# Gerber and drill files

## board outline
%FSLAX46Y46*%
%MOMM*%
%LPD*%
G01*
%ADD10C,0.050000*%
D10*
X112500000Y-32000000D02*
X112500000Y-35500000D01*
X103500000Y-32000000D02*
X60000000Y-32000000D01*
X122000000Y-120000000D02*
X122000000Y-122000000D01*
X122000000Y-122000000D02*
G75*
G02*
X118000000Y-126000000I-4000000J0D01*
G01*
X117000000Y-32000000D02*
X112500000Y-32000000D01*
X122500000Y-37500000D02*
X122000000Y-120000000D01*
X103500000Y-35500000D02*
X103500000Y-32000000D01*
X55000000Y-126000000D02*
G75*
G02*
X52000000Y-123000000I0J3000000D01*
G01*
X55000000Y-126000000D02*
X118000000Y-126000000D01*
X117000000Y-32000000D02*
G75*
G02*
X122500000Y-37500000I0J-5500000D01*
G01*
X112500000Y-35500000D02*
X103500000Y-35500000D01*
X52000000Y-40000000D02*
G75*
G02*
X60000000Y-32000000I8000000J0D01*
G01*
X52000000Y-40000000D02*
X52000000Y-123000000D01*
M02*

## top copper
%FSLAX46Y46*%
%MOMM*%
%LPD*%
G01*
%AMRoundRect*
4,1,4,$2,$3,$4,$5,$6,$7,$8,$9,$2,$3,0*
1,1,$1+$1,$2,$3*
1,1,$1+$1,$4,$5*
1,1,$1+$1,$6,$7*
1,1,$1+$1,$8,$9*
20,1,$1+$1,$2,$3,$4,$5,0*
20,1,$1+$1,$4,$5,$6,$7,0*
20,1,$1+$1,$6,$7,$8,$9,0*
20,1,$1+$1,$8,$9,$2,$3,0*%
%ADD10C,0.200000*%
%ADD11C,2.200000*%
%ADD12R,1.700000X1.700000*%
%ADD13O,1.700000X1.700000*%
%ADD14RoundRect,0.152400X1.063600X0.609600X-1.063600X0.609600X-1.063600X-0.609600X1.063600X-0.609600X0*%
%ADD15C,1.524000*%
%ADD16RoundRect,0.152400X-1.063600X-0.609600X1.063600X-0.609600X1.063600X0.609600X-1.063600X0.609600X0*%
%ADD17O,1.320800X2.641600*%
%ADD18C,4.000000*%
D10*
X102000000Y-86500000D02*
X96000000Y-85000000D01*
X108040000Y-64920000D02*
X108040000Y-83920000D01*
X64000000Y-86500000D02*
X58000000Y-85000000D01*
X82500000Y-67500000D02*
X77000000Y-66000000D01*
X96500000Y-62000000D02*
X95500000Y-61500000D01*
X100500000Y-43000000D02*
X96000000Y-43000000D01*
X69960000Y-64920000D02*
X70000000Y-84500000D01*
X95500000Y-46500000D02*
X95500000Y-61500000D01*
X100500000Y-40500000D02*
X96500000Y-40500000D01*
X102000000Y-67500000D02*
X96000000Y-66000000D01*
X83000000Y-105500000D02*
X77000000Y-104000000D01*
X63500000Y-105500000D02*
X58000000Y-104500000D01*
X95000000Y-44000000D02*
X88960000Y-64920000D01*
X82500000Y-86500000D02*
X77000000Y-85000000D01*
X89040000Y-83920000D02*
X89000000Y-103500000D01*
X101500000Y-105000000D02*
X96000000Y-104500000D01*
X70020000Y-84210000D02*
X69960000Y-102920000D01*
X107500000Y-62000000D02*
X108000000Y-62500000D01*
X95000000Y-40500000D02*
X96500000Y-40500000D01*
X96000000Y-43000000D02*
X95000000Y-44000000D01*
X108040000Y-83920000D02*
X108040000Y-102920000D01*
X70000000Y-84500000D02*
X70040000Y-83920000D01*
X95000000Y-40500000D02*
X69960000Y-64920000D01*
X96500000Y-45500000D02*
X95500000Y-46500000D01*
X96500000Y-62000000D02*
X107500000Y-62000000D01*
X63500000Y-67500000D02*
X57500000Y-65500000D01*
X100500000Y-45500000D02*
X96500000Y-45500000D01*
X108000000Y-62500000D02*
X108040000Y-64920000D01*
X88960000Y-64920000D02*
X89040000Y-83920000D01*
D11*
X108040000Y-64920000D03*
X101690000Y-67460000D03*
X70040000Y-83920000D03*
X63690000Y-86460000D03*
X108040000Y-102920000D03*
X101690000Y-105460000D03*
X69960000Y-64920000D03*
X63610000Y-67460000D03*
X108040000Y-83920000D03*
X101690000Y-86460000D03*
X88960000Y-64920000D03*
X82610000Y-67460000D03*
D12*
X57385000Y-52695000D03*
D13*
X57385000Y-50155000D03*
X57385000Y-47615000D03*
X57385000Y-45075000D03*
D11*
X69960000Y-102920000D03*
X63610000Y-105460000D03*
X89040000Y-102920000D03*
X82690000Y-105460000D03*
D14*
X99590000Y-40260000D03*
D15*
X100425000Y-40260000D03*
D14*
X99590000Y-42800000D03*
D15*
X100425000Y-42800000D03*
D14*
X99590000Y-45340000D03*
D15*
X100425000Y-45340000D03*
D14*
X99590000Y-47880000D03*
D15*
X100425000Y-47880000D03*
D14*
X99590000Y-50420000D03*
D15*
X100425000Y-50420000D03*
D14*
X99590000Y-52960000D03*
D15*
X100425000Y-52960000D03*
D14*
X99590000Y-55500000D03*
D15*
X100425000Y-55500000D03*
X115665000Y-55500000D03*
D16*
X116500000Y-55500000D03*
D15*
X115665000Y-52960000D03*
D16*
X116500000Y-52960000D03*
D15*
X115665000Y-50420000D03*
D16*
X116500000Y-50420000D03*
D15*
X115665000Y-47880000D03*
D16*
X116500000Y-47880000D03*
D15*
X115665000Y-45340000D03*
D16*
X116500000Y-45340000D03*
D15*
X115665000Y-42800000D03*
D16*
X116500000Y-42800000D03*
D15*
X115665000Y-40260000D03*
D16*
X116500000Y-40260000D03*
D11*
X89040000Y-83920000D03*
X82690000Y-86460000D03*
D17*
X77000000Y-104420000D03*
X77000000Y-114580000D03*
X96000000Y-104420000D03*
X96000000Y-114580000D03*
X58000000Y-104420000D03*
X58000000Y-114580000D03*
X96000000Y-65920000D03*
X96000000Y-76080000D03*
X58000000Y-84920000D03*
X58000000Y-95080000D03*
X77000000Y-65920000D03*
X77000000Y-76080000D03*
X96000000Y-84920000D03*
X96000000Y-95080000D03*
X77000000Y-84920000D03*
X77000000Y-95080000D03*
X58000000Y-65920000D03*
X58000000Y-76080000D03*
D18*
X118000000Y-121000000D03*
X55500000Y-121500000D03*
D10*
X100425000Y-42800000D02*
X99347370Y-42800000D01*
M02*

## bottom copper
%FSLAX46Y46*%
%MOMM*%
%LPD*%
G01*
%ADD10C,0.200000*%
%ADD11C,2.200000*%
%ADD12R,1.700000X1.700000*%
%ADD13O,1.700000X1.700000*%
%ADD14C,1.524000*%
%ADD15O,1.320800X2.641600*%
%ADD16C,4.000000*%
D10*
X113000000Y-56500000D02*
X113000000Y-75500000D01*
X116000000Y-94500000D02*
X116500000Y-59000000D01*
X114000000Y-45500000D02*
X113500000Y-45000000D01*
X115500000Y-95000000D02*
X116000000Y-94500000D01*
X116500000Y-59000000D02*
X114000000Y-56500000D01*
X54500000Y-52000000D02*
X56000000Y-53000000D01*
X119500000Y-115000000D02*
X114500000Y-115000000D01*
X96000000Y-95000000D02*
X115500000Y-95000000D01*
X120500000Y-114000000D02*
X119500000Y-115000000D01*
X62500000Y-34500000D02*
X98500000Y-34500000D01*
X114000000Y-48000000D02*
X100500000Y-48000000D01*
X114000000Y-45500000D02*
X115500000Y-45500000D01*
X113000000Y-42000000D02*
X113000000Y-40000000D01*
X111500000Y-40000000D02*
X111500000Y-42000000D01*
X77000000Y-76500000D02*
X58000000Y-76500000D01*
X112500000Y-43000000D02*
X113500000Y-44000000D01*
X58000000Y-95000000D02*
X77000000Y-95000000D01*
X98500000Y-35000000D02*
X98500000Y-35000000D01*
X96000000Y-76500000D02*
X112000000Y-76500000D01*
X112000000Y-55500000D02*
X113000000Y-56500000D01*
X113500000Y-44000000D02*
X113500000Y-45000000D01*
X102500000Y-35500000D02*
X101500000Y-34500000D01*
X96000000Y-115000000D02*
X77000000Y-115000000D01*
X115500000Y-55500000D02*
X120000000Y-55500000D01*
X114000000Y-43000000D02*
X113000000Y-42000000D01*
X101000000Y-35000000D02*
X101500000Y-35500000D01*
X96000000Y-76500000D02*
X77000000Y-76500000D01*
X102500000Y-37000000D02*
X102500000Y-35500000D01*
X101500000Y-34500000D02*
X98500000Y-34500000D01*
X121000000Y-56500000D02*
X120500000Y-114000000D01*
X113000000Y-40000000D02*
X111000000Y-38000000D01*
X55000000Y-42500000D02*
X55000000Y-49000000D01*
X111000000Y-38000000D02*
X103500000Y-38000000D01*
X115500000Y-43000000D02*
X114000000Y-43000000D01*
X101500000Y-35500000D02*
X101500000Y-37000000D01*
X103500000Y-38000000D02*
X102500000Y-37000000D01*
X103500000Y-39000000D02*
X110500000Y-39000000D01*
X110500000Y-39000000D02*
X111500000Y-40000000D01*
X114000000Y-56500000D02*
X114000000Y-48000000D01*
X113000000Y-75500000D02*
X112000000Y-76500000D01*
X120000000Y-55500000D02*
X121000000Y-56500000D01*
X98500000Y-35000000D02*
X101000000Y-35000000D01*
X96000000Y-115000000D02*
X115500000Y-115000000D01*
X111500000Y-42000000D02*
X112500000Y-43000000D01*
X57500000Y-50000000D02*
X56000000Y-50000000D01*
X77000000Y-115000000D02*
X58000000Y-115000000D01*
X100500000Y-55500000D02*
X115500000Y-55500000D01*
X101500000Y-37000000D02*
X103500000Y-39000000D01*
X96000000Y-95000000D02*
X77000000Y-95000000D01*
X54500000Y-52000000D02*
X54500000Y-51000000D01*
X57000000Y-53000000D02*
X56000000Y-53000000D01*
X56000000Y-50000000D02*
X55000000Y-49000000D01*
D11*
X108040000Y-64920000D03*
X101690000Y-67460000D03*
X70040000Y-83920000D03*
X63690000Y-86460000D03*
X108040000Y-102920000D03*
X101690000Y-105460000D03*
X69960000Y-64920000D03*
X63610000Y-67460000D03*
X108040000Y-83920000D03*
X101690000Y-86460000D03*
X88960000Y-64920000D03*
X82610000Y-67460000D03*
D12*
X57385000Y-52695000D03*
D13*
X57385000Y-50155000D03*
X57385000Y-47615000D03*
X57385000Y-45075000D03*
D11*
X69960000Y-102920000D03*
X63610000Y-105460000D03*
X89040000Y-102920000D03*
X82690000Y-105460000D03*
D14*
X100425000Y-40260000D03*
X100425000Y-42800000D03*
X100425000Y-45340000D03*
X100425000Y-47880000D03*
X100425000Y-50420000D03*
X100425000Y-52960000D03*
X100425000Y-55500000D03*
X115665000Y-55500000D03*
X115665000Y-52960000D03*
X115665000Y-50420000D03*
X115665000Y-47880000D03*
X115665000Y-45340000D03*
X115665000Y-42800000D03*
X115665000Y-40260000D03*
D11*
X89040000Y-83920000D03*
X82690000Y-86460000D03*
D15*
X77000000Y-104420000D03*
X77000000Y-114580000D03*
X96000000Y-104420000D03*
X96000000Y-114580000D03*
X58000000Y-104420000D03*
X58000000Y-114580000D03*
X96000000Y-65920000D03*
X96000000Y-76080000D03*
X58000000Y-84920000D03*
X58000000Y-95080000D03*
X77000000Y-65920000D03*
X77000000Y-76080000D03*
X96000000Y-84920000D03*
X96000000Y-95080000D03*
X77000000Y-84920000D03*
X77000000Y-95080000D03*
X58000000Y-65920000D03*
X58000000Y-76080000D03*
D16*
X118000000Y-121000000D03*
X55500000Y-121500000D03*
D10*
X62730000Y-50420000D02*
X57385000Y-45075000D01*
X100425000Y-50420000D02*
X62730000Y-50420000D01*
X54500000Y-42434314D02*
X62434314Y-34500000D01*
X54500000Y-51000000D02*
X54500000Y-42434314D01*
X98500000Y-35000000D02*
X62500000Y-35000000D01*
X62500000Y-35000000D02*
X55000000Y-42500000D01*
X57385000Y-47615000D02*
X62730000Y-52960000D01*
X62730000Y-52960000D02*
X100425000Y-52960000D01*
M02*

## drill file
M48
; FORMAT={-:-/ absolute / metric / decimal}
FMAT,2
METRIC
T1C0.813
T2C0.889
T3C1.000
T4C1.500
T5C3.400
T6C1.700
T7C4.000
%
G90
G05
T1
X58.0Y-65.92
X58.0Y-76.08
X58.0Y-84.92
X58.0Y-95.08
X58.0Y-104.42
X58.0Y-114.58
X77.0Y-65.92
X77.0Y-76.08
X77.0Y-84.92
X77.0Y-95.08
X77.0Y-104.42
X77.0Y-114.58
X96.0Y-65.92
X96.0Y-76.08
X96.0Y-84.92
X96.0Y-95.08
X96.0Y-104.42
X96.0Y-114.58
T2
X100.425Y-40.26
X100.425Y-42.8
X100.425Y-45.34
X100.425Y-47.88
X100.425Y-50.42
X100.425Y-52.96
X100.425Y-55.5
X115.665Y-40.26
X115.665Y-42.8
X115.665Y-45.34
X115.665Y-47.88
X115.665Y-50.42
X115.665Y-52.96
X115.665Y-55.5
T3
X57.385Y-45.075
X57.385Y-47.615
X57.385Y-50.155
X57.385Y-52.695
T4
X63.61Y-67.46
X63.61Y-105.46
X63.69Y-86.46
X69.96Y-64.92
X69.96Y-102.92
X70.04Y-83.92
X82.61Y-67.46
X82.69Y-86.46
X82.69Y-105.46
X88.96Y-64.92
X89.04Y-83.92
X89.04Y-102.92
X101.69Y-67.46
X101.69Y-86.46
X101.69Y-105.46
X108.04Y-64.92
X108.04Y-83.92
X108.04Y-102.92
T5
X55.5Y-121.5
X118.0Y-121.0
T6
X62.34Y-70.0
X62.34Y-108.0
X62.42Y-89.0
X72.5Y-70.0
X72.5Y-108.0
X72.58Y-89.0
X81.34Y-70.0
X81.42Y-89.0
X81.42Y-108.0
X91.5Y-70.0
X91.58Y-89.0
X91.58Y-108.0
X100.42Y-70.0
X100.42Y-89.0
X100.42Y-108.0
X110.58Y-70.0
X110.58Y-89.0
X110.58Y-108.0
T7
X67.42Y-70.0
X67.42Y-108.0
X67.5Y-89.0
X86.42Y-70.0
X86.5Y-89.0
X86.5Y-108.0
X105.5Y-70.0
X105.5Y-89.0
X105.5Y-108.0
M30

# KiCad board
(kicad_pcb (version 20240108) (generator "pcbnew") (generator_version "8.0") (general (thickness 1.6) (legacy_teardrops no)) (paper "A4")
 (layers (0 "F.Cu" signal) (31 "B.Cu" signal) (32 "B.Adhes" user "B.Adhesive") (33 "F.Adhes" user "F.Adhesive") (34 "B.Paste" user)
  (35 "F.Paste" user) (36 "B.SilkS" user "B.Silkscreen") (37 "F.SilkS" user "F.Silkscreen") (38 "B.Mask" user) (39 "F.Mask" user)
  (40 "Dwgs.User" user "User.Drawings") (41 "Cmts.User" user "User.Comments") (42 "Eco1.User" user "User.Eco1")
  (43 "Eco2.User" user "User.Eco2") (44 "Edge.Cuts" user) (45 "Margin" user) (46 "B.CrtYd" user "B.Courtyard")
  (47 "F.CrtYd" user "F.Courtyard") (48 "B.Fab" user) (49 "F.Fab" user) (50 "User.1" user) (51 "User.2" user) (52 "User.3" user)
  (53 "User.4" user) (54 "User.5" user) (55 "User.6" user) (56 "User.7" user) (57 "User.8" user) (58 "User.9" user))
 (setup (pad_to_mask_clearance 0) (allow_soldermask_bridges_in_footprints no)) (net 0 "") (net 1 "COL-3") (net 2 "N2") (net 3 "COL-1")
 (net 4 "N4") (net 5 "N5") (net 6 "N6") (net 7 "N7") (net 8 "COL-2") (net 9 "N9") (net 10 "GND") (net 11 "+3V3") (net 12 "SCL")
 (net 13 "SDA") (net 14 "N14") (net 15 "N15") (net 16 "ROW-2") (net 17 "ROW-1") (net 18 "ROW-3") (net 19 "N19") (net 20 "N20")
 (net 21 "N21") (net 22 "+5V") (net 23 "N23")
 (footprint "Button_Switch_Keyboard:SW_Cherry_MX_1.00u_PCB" (layer "F.Cu") (at 108.04 64.92)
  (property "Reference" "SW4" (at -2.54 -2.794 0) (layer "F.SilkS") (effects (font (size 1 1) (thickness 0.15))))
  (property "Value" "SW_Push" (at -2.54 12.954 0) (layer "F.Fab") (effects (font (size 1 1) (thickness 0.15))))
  (pad "" np_thru_hole circle (at -7.62 5.08) (size 1.7 1.7) (drill 1.7) (layers "*.Cu" "*.Mask"))
  (pad "" np_thru_hole circle (at -2.54 5.08) (size 4 4) (drill 4) (layers "*.Cu" "*.Mask"))
  (pad "" np_thru_hole circle (at 2.54 5.08) (size 1.7 1.7) (drill 1.7) (layers "*.Cu" "*.Mask"))
  (pad "1" thru_hole circle (at 0 0) (size 2.2 2.2) (drill 1.5) (layers "*.Cu" "*.Mask") (remove_unused_layers no) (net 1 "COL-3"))
  (pad "2" thru_hole circle (at -6.35 2.54) (size 2.2 2.2) (drill 1.5) (layers "*.Cu" "*.Mask") (remove_unused_layers no) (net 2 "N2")))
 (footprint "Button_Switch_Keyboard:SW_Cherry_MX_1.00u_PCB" (layer "F.Cu") (at 70.04 83.92)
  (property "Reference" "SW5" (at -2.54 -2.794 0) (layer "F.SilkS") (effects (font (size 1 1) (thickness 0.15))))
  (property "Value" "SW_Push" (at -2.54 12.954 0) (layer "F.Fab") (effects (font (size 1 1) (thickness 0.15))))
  (pad "" np_thru_hole circle (at -7.62 5.08) (size 1.7 1.7) (drill 1.7) (layers "*.Cu" "*.Mask"))
  (pad "" np_thru_hole circle (at -2.54 5.08) (size 4 4) (drill 4) (layers "*.Cu" "*.Mask"))
  (pad "" np_thru_hole circle (at 2.54 5.08) (size 1.7 1.7) (drill 1.7) (layers "*.Cu" "*.Mask"))
  (pad "1" thru_hole circle (at 0 0) (size 2.2 2.2) (drill 1.5) (layers "*.Cu" "*.Mask") (remove_unused_layers no) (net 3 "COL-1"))
  (pad "2" thru_hole circle (at -6.35 2.54) (size 2.2 2.2) (drill 1.5) (layers "*.Cu" "*.Mask") (remove_unused_layers no) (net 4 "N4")))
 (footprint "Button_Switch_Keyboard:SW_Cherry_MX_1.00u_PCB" (layer "F.Cu") (at 108.04 102.92)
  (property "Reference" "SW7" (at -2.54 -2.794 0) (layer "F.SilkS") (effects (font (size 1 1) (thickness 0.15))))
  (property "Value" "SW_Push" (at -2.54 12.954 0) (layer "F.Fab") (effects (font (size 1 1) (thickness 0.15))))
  (pad "" np_thru_hole circle (at -7.62 5.08) (size 1.7 1.7) (drill 1.7) (layers "*.Cu" "*.Mask"))
  (pad "" np_thru_hole circle (at -2.54 5.08) (size 4 4) (drill 4) (layers "*.Cu" "*.Mask"))
  (pad "" np_thru_hole circle (at 2.54 5.08) (size 1.7 1.7) (drill 1.7) (layers "*.Cu" "*.Mask"))
  (pad "1" thru_hole circle (at 0 0) (size 2.2 2.2) (drill 1.5) (layers "*.Cu" "*.Mask") (remove_unused_layers no) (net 1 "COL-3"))
  (pad "2" thru_hole circle (at -6.35 2.54) (size 2.2 2.2) (drill 1.5) (layers "*.Cu" "*.Mask") (remove_unused_layers no) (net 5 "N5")))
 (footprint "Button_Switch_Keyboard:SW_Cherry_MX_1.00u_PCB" (layer "F.Cu") (at 69.96 64.92)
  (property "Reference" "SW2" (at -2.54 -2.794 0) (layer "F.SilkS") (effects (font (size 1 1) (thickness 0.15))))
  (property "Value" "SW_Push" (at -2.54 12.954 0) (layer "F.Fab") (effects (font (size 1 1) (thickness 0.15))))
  (pad "" np_thru_hole circle (at -7.62 5.08) (size 1.7 1.7) (drill 1.7) (layers "*.Cu" "*.Mask"))
  (pad "" np_thru_hole circle (at -2.54 5.08) (size 4 4) (drill 4) (layers "*.Cu" "*.Mask"))
  (pad "" np_thru_hole circle (at 2.54 5.08) (size 1.7 1.7) (drill 1.7) (layers "*.Cu" "*.Mask"))
  (pad "1" thru_hole circle (at 0 0) (size 2.2 2.2) (drill 1.5) (layers "*.Cu" "*.Mask") (remove_unused_layers no) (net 3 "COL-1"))
  (pad "2" thru_hole circle (at -6.35 2.54) (size 2.2 2.2) (drill 1.5) (layers "*.Cu" "*.Mask") (remove_unused_layers no) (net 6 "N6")))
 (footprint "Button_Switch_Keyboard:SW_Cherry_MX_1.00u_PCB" (layer "F.Cu") (at 108.04 83.92)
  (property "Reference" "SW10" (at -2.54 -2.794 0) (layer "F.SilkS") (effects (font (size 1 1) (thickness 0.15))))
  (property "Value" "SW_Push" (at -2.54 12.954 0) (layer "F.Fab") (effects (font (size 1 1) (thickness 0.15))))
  (pad "" np_thru_hole circle (at -7.62 5.08) (size 1.7 1.7) (drill 1.7) (layers "*.Cu" "*.Mask"))
  (pad "" np_thru_hole circle (at -2.54 5.08) (size 4 4) (drill 4) (layers "*.Cu" "*.Mask"))
  (pad "" np_thru_hole circle (at 2.54 5.08) (size 1.7 1.7) (drill 1.7) (layers "*.Cu" "*.Mask"))
  (pad "1" thru_hole circle (at 0 0) (size 2.2 2.2) (drill 1.5) (layers "*.Cu" "*.Mask") (remove_unused_layers no) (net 1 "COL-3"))
  (pad "2" thru_hole circle (at -6.35 2.54) (size 2.2 2.2) (drill 1.5) (layers "*.Cu" "*.Mask") (remove_unused_layers no) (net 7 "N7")))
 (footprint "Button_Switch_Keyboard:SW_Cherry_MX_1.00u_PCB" (layer "F.Cu") (at 88.96 64.92)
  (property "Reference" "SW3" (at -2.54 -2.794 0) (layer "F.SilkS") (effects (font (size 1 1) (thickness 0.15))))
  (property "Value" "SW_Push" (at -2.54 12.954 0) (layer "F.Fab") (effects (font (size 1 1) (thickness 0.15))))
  (pad "" np_thru_hole circle (at -7.62 5.08) (size 1.7 1.7) (drill 1.7) (layers "*.Cu" "*.Mask"))
  (pad "" np_thru_hole circle (at -2.54 5.08) (size 4 4) (drill 4) (layers "*.Cu" "*.Mask"))
  (pad "" np_thru_hole circle (at 2.54 5.08) (size 1.7 1.7) (drill 1.7) (layers "*.Cu" "*.Mask"))
  (pad "1" thru_hole circle (at 0 0) (size 2.2 2.2) (drill 1.5) (layers "*.Cu" "*.Mask") (remove_unused_layers no) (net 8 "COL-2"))
  (pad "2" thru_hole circle (at -6.35 2.54) (size 2.2 2.2) (drill 1.5) (layers "*.Cu" "*.Mask") (remove_unused_layers no) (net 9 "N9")))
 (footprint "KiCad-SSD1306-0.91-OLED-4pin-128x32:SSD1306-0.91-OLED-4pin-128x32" (layer "F.Cu") (at 93.885 54.885 180)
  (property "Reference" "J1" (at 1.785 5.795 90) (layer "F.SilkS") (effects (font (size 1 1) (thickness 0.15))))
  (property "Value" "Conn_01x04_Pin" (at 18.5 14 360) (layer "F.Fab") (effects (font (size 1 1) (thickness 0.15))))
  (pad "1" thru_hole rect (at 36.5 2.19 180) (size 1.7 1.7) (drill 1) (layers "*.Cu" "*.Mask") (remove_unused_layers no) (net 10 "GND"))
  (pad "2" thru_hole oval (at 36.5 4.73 180) (size 1.7 1.7) (drill 1) (layers "*.Cu" "*.Mask") (remove_unused_layers no) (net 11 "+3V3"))
  (pad "3" thru_hole oval (at 36.5 7.27 180) (size 1.7 1.7) (drill 1) (layers "*.Cu" "*.Mask") (remove_unused_layers no) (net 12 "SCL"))
  (pad "4" thru_hole oval (at 36.5 9.81 180) (size 1.7 1.7) (drill 1) (layers "*.Cu" "*.Mask") (remove_unused_layers no) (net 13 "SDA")))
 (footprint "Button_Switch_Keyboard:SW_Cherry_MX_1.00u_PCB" (layer "F.Cu") (at 69.96 102.92)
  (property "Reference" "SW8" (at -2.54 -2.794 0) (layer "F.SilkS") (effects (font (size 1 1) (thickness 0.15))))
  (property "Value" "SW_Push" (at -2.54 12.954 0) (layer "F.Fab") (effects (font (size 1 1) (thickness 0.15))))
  (pad "" np_thru_hole circle (at -7.62 5.08) (size 1.7 1.7) (drill 1.7) (layers "*.Cu" "*.Mask"))
  (pad "" np_thru_hole circle (at -2.54 5.08) (size 4 4) (drill 4) (layers "*.Cu" "*.Mask"))
  (pad "" np_thru_hole circle (at 2.54 5.08) (size 1.7 1.7) (drill 1.7) (layers "*.Cu" "*.Mask"))
  (pad "1" thru_hole circle (at 0 0) (size 2.2 2.2) (drill 1.5) (layers "*.Cu" "*.Mask") (remove_unused_layers no) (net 3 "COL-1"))
  (pad "2" thru_hole circle (at -6.35 2.54) (size 2.2 2.2) (drill 1.5) (layers "*.Cu" "*.Mask") (remove_unused_layers no) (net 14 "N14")))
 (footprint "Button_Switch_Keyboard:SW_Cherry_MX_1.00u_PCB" (layer "F.Cu") (at 89.04 102.92)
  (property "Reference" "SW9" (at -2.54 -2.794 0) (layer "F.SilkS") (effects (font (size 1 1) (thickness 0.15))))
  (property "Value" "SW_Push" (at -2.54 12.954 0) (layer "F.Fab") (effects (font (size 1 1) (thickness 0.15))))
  (pad "" np_thru_hole circle (at -7.62 5.08) (size 1.7 1.7) (drill 1.7) (layers "*.Cu" "*.Mask"))
  (pad "" np_thru_hole circle (at -2.54 5.08) (size 4 4) (drill 4) (layers "*.Cu" "*.Mask"))
  (pad "" np_thru_hole circle (at 2.54 5.08) (size 1.7 1.7) (drill 1.7) (layers "*.Cu" "*.Mask"))
  (pad "1" thru_hole circle (at 0 0) (size 2.2 2.2) (drill 1.5) (layers "*.Cu" "*.Mask") (remove_unused_layers no) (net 8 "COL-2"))
  (pad "2" thru_hole circle (at -6.35 2.54) (size 2.2 2.2) (drill 1.5) (layers "*.Cu" "*.Mask") (remove_unused_layers no) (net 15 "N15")))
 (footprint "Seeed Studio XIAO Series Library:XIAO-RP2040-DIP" (layer "F.Cu") (at 108.045 47.88)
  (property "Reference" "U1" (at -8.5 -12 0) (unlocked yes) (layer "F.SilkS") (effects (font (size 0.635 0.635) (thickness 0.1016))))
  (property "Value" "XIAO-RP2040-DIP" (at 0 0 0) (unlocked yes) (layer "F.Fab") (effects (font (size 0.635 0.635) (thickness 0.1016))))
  (pad "1" smd roundrect (at -8.455 -7.62 180) (size 2.432 1.524) (layers "F.Cu" "F.Mask") (roundrect_rratio 0.1) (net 3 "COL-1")
   (thermal_bridge_angle 45))
  (pad "1" thru_hole circle (at -7.62 -7.62 180) (size 1.524 1.524) (drill 0.889) (layers "*.Cu" "*.Mask") (remove_unused_layers no)
   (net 3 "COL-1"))
  (pad "2" smd roundrect (at -8.455 -5.08 180) (size 2.432 1.524) (layers "F.Cu" "F.Mask") (roundrect_rratio 0.1) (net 8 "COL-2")
   (thermal_bridge_angle 45))
  (pad "2" thru_hole circle (at -7.62 -5.08 180) (size 1.524 1.524) (drill 0.889) (layers "*.Cu" "*.Mask") (remove_unused_layers no)
   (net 8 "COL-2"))
  (pad "3" smd roundrect (at -8.455 -2.54 180) (size 2.432 1.524) (layers "F.Cu" "F.Mask") (roundrect_rratio 0.1) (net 1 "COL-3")
   (thermal_bridge_angle 45))
  (pad "3" thru_hole circle (at -7.62 -2.54 180) (size 1.524 1.524) (drill 0.889) (layers "*.Cu" "*.Mask") (remove_unused_layers no)
   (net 1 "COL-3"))
  (pad "4" smd roundrect (at -8.455 0 180) (size 2.432 1.524) (layers "F.Cu" "F.Mask") (roundrect_rratio 0.1) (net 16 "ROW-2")
   (thermal_bridge_angle 45))
  (pad "4" thru_hole circle (at -7.62 0 180) (size 1.524 1.524) (drill 0.889) (layers "*.Cu" "*.Mask") (remove_unused_layers no)
   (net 16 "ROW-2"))
  (pad "5" smd roundrect (at -8.455 2.54 180) (size 2.432 1.524) (layers "F.Cu" "F.Mask") (roundrect_rratio 0.1) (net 13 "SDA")
   (thermal_bridge_angle 45))
  (pad "5" thru_hole circle (at -7.62 2.54 180) (size 1.524 1.524) (drill 0.889) (layers "*.Cu" "*.Mask") (remove_unused_layers no)
   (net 13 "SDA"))
  (pad "6" smd roundrect (at -8.455 5.08 180) (size 2.432 1.524) (layers "F.Cu" "F.Mask") (roundrect_rratio 0.1) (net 12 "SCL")
   (thermal_bridge_angle 45))
  (pad "6" thru_hole circle (at -7.62 5.08 180) (size 1.524 1.524) (drill 0.889) (layers "*.Cu" "*.Mask") (remove_unused_layers no)
   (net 12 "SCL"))
  (pad "7" smd roundrect (at -8.455 7.62 180) (size 2.432 1.524) (layers "F.Cu" "F.Mask") (roundrect_rratio 0.1) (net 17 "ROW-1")
   (thermal_bridge_angle 45))
  (pad "7" thru_hole circle (at -7.62 7.62 180) (size 1.524 1.524) (drill 0.889) (layers "*.Cu" "*.Mask") (remove_unused_layers no)
   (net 17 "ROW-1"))
  (pad "8" thru_hole circle (at 7.62 7.62) (size 1.524 1.524) (drill 0.889) (layers "*.Cu" "*.Mask") (remove_unused_layers no)
   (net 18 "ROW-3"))
  (pad "8" smd roundrect (at 8.455 7.62) (size 2.432 1.524) (layers "F.Cu" "F.Mask") (roundrect_rratio 0.1) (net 18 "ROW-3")
   (thermal_bridge_angle 45))
  (pad "9" thru_hole circle (at 7.62 5.08) (size 1.524 1.524) (drill 0.889) (layers "*.Cu" "*.Mask") (remove_unused_layers no)
   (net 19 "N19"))
  (pad "9" smd roundrect (at 8.455 5.08) (size 2.432 1.524) (layers "F.Cu" "F.Mask") (roundrect_rratio 0.1) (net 19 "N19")
   (thermal_bridge_angle 45))
  (pad "10" thru_hole circle (at 7.62 2.54) (size 1.524 1.524) (drill 0.889) (layers "*.Cu" "*.Mask") (remove_unused_layers no)
   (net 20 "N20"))
  (pad "10" smd roundrect (at 8.455 2.54) (size 2.432 1.524) (layers "F.Cu" "F.Mask") (roundrect_rratio 0.1) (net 20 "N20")
   (thermal_bridge_angle 45))
  (pad "11" thru_hole circle (at 7.62 0) (size 1.524 1.524) (drill 0.889) (layers "*.Cu" "*.Mask") (remove_unused_layers no) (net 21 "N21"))
  (pad "11" smd roundrect (at 8.455 0) (size 2.432 1.524) (layers "F.Cu" "F.Mask") (roundrect_rratio 0.1) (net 21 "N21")
   (thermal_bridge_angle 45))
  (pad "12" thru_hole circle (at 7.62 -2.54) (size 1.524 1.524) (drill 0.889) (layers "*.Cu" "*.Mask") (remove_unused_layers no)
   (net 11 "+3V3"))
  (pad "12" smd roundrect (at 8.455 -2.54) (size 2.432 1.524) (layers "F.Cu" "F.Mask") (roundrect_rratio 0.1) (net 11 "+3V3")
   (thermal_bridge_angle 45))
  (pad "13" thru_hole circle (at 7.62 -5.08) (size 1.524 1.524) (drill 0.889) (layers "*.Cu" "*.Mask") (remove_unused_layers no)
   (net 10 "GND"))
  (pad "13" smd roundrect (at 8.455 -5.08) (size 2.432 1.524) (layers "F.Cu" "F.Mask") (roundrect_rratio 0.1) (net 10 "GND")
   (thermal_bridge_angle 45))
  (pad "14" thru_hole circle (at 7.62 -7.62) (size 1.524 1.524) (drill 0.889) (layers "*.Cu" "*.Mask") (remove_unused_layers no)
   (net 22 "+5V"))
  (pad "14" smd roundrect (at 8.455 -7.62) (size 2.432 1.524) (layers "F.Cu" "F.Mask") (roundrect_rratio 0.1) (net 22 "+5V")
   (thermal_bridge_angle 45)))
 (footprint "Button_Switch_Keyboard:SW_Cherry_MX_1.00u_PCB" (layer "F.Cu") (at 89.04 83.92)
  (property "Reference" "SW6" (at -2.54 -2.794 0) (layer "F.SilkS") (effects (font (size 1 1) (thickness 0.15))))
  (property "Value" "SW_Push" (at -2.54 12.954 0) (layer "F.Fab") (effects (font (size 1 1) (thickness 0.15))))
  (pad "" np_thru_hole circle (at -7.62 5.08) (size 1.7 1.7) (drill 1.7) (layers "*.Cu" "*.Mask"))
  (pad "" np_thru_hole circle (at -2.54 5.08) (size 4 4) (drill 4) (layers "*.Cu" "*.Mask"))
  (pad "" np_thru_hole circle (at 2.54 5.08) (size 1.7 1.7) (drill 1.7) (layers "*.Cu" "*.Mask"))
  (pad "1" thru_hole circle (at 0 0) (size 2.2 2.2) (drill 1.5) (layers "*.Cu" "*.Mask") (remove_unused_layers no) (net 8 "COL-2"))
  (pad "2" thru_hole circle (at -6.35 2.54) (size 2.2 2.2) (drill 1.5) (layers "*.Cu" "*.Mask") (remove_unused_layers no) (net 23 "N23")))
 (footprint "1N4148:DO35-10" (layer "B.Cu") (at 77 109.5 90)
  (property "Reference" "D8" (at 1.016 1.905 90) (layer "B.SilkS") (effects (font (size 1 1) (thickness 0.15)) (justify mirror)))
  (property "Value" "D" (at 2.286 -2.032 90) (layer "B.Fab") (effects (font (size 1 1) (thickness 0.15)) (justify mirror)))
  (pad "A" thru_hole oval (at 5.08 0 90) (size 2.6416 1.3208) (drill 0.8128) (layers "*.Cu" "*.Mask") (remove_unused_layers no)
   (solder_mask_margin 0.102))
  (pad "C" thru_hole oval (at -5.08 0 90) (size 2.6416 1.3208) (drill 0.8128) (layers "*.Cu" "*.Mask") (remove_unused_layers no)
   (solder_mask_margin 0.102)))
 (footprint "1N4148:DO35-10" (layer "B.Cu") (at 96 109.5 90)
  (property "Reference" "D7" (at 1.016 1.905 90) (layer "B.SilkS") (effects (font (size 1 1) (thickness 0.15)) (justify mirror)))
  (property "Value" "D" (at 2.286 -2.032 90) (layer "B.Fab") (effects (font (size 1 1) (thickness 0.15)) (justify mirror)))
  (pad "A" thru_hole oval (at 5.08 0 90) (size 2.6416 1.3208) (drill 0.8128) (layers "*.Cu" "*.Mask") (remove_unused_layers no)
   (solder_mask_margin 0.102))
  (pad "C" thru_hole oval (at -5.08 0 90) (size 2.6416 1.3208) (drill 0.8128) (layers "*.Cu" "*.Mask") (remove_unused_layers no)
   (solder_mask_margin 0.102)))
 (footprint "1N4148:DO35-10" (layer "B.Cu") (at 58 109.5 90)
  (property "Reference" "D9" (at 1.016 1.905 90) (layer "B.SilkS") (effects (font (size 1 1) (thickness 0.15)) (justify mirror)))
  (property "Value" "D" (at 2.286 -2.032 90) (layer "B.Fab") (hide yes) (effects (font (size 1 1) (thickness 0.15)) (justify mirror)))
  (pad "A" thru_hole oval (at 5.08 0 90) (size 2.6416 1.3208) (drill 0.8128) (layers "*.Cu" "*.Mask") (remove_unused_layers no)
   (solder_mask_margin 0.102))
  (pad "C" thru_hole oval (at -5.08 0 90) (size 2.6416 1.3208) (drill 0.8128) (layers "*.Cu" "*.Mask") (remove_unused_layers no)
   (solder_mask_margin 0.102)))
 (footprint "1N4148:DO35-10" (layer "B.Cu") (at 96 71 90)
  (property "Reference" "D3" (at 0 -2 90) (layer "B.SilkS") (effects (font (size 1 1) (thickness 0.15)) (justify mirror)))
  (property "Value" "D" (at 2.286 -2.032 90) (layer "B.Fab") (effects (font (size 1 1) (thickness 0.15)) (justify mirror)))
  (pad "A" thru_hole oval (at 5.08 0 90) (size 2.6416 1.3208) (drill 0.8128) (layers "*.Cu" "*.Mask") (remove_unused_layers no)
   (solder_mask_margin 0.102))
  (pad "C" thru_hole oval (at -5.08 0 90) (size 2.6416 1.3208) (drill 0.8128) (layers "*.Cu" "*.Mask") (remove_unused_layers no)
   (solder_mask_margin 0.102)))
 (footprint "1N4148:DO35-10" (layer "B.Cu") (at 58 90 90)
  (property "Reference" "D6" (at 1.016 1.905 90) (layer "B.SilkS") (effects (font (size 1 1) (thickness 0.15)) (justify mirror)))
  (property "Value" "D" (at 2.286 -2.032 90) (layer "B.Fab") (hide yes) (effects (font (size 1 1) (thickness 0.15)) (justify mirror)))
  (pad "A" thru_hole oval (at 5.08 0 90) (size 2.6416 1.3208) (drill 0.8128) (layers "*.Cu" "*.Mask") (remove_unused_layers no)
   (solder_mask_margin 0.102))
  (pad "C" thru_hole oval (at -5.08 0 90) (size 2.6416 1.3208) (drill 0.8128) (layers "*.Cu" "*.Mask") (remove_unused_layers no)
   (solder_mask_margin 0.102)))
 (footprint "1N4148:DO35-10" (layer "B.Cu") (at 77 71 90)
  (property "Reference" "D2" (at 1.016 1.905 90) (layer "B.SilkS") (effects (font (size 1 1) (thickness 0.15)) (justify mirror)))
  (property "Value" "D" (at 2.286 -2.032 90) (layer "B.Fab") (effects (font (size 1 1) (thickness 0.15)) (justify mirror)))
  (pad "A" thru_hole oval (at 5.08 0 90) (size 2.6416 1.3208) (drill 0.8128) (layers "*.Cu" "*.Mask") (remove_unused_layers no)
   (solder_mask_margin 0.102))
  (pad "C" thru_hole oval (at -5.08 0 90) (size 2.6416 1.3208) (drill 0.8128) (layers "*.Cu" "*.Mask") (remove_unused_layers no)
   (solder_mask_margin 0.102)))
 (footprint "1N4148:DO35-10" (layer "B.Cu") (at 96 90 90)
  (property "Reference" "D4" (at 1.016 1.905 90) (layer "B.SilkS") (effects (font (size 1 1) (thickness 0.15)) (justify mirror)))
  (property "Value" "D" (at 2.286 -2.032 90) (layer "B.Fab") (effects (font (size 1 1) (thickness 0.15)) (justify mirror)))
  (pad "A" thru_hole oval (at 5.08 0 90) (size 2.6416 1.3208) (drill 0.8128) (layers "*.Cu" "*.Mask") (remove_unused_layers no)
   (solder_mask_margin 0.102))
  (pad "C" thru_hole oval (at -5.08 0 90) (size 2.6416 1.3208) (drill 0.8128) (layers "*.Cu" "*.Mask") (remove_unused_layers no)
   (solder_mask_margin 0.102)))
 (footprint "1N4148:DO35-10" (layer "B.Cu") (at 77 90 90)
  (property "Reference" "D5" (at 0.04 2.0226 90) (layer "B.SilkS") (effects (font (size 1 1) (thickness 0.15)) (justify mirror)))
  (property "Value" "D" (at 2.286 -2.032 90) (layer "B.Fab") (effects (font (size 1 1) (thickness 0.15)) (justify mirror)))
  (pad "A" thru_hole oval (at 5.08 0 90) (size 2.6416 1.3208) (drill 0.8128) (layers "*.Cu" "*.Mask") (remove_unused_layers no)
   (solder_mask_margin 0.102))
  (pad "C" thru_hole oval (at -5.08 0 90) (size 2.6416 1.3208) (drill 0.8128) (layers "*.Cu" "*.Mask") (remove_unused_layers no)
   (solder_mask_margin 0.102)))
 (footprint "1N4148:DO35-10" (layer "B.Cu") (at 58 71 90)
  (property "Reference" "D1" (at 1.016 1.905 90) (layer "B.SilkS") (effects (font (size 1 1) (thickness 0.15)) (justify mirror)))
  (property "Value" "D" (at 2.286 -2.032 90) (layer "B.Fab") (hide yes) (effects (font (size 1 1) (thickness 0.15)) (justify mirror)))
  (pad "A" thru_hole oval (at 5.08 0 90) (size 2.6416 1.3208) (drill 0.8128) (layers "*.Cu" "*.Mask") (remove_unused_layers no)
   (solder_mask_margin 0.102))
  (pad "C" thru_hole oval (at -5.08 0 90) (size 2.6416 1.3208) (drill 0.8128) (layers "*.Cu" "*.Mask") (remove_unused_layers no)
   (solder_mask_margin 0.102)))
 (gr_line (start 102 86.5) (end 96 85) (stroke (width 0.2) (type default)) (layer "F.Cu") (net 7))
 (gr_line (start 108.04 64.92) (end 108.04 83.92) (stroke (width 0.2) (type default)) (layer "F.Cu") (net 1))
 (gr_line (start 64 86.5) (end 58 85) (stroke (width 0.2) (type default)) (layer "F.Cu") (net 4))
 (gr_line (start 82.5 67.5) (end 77 66) (stroke (width 0.2) (type default)) (layer "F.Cu") (net 9))
 (gr_line (start 96.5 62) (end 95.5 61.5) (stroke (width 0.2) (type default)) (layer "F.Cu") (net 1))
 (gr_line (start 100.5 43) (end 96 43) (stroke (width 0.2) (type default)) (layer "F.Cu") (net 8))
 (gr_line (start 69.96 64.92) (end 70 84.5) (stroke (width 0.2) (type default)) (layer "F.Cu") (net 3))
 (gr_line (start 95.5 46.5) (end 95.5 61.5) (stroke (width 0.2) (type default)) (layer "F.Cu") (net 1))
 (gr_line (start 100.5 40.5) (end 96.5 40.5) (stroke (width 0.2) (type default)) (layer "F.Cu") (net 3))
 (gr_line (start 102 67.5) (end 96 66) (stroke (width 0.2) (type default)) (layer "F.Cu") (net 2))
 (gr_line (start 83 105.5) (end 77 104) (stroke (width 0.2) (type default)) (layer "F.Cu") (net 15))
 (gr_line (start 63.5 105.5) (end 58 104.5) (stroke (width 0.2) (type default)) (layer "F.Cu") (net 14))
 (gr_line (start 95 44) (end 88.96 64.92) (stroke (width 0.2) (type default)) (layer "F.Cu") (net 8))
 (gr_line (start 82.5 86.5) (end 77 85) (stroke (width 0.2) (type default)) (layer "F.Cu") (net 23))
 (gr_line (start 89.04 83.92) (end 89 103.5) (stroke (width 0.2) (type default)) (layer "F.Cu") (net 8))
 (gr_line (start 101.5 105) (end 96 104.5) (stroke (width 0.2) (type default)) (layer "F.Cu") (net 5))
 (gr_line (start 70.02 84.21) (end 69.96 102.92) (stroke (width 0.2) (type default)) (layer "F.Cu") (net 3))
 (gr_line (start 107.5 62) (end 108 62.5) (stroke (width 0.2) (type default)) (layer "F.Cu") (net 1))
 (gr_line (start 95 40.5) (end 96.5 40.5) (stroke (width 0.2) (type default)) (layer "F.Cu") (net 3))
 (gr_line (start 96 43) (end 95 44) (stroke (width 0.2) (type default)) (layer "F.Cu") (net 8))
 (gr_line (start 108.04 83.92) (end 108.04 102.92) (stroke (width 0.2) (type default)) (layer "F.Cu") (net 1))
 (gr_line (start 70 84.5) (end 70.04 83.92) (stroke (width 0.2) (type default)) (layer "F.Cu") (net 3))
 (gr_line (start 95 40.5) (end 69.96 64.92) (stroke (width 0.2) (type default)) (layer "F.Cu") (net 3))
 (gr_line (start 96.5 45.5) (end 95.5 46.5) (stroke (width 0.2) (type default)) (layer "F.Cu") (net 1))
 (gr_line (start 96.5 62) (end 107.5 62) (stroke (width 0.2) (type default)) (layer "F.Cu") (net 1))
 (gr_line (start 63.5 67.5) (end 57.5 65.5) (stroke (width 0.2) (type default)) (layer "F.Cu") (net 6))
 (gr_line (start 100.5 45.5) (end 96.5 45.5) (stroke (width 0.2) (type default)) (layer "F.Cu") (net 1))
 (gr_line (start 108 62.5) (end 108.04 64.92) (stroke (width 0.2) (type default)) (layer "F.Cu") (net 1))
 (gr_line (start 88.96 64.92) (end 89.04 83.92) (stroke (width 0.2) (type default)) (layer "F.Cu") (net 8))
 (gr_line (start 113 56.5) (end 113 75.5) (stroke (width 0.2) (type default)) (layer "B.Cu") (net 17))
 (gr_line (start 116 94.5) (end 116.5 59) (stroke (width 0.2) (type default)) (layer "B.Cu") (net 16))
 (gr_line (start 114 45.5) (end 113.5 45) (stroke (width 0.2) (type default)) (layer "B.Cu") (net 11))
 (gr_line (start 115.5 95) (end 116 94.5) (stroke (width 0.2) (type default)) (layer "B.Cu") (net 16))
 (gr_line (start 116.5 59) (end 114 56.5) (stroke (width 0.2) (type default)) (layer "B.Cu") (net 16))
 (gr_line (start 54.5 52) (end 56 53) (stroke (width 0.2) (type default)) (layer "B.Cu") (net 10))
 (gr_line (start 119.5 115) (end 114.5 115) (stroke (width 0.2) (type default)) (layer "B.Cu") (net 18))
 (gr_line (start 96 95) (end 115.5 95) (stroke (width 0.2) (type default)) (layer "B.Cu") (net 16))
 (gr_line (start 120.5 114) (end 119.5 115) (stroke (width 0.2) (type default)) (layer "B.Cu") (net 18))
 (gr_line (start 62.5 34.5) (end 98.5 34.5) (stroke (width 0.2) (type default)) (layer "B.Cu") (net 10))
 (gr_line (start 114 48) (end 100.5 48) (stroke (width 0.2) (type default)) (layer "B.Cu") (net 16))
 (gr_line (start 114 45.5) (end 115.5 45.5) (stroke (width 0.2) (type default)) (layer "B.Cu") (net 11))
 (gr_line (start 113 42) (end 113 40) (stroke (width 0.2) (type default)) (layer "B.Cu") (net 10))
 (gr_line (start 111.5 40) (end 111.5 42) (stroke (width 0.2) (type default)) (layer "B.Cu") (net 11))
 (gr_line (start 77 76.5) (end 58 76.5) (stroke (width 0.2) (type default)) (layer "B.Cu") (net 17))
 (gr_line (start 112.5 43) (end 113.5 44) (stroke (width 0.2) (type default)) (layer "B.Cu") (net 11))
 (gr_line (start 58 95) (end 77 95) (stroke (width 0.2) (type default)) (layer "B.Cu") (net 16))
 (gr_line (start 98.5 35) (end 98.5 35) (stroke (width 0.2) (type default)) (layer "B.Cu") (net 11))
 (gr_line (start 96 76.5) (end 112 76.5) (stroke (width 0.2) (type default)) (layer "B.Cu") (net 17))
 (gr_line (start 112 55.5) (end 113 56.5) (stroke (width 0.2) (type default)) (layer "B.Cu") (net 17))
 (gr_line (start 113.5 44) (end 113.5 45) (stroke (width 0.2) (type default)) (layer "B.Cu") (net 11))
 (gr_line (start 102.5 35.5) (end 101.5 34.5) (stroke (width 0.2) (type default)) (layer "B.Cu") (net 10))
 (gr_line (start 96 115) (end 77 115) (stroke (width 0.2) (type default)) (layer "B.Cu") (net 18))
 (gr_line (start 115.5 55.5) (end 120 55.5) (stroke (width 0.2) (type default)) (layer "B.Cu") (net 18))
 (gr_line (start 114 43) (end 113 42) (stroke (width 0.2) (type default)) (layer "B.Cu") (net 10))
 (gr_line (start 101 35) (end 101.5 35.5) (stroke (width 0.2) (type default)) (layer "B.Cu") (net 11))
 (gr_line (start 96 76.5) (end 77 76.5) (stroke (width 0.2) (type default)) (layer "B.Cu") (net 17))
 (gr_line (start 102.5 37) (end 102.5 35.5) (stroke (width 0.2) (type default)) (layer "B.Cu") (net 10))
 (gr_line (start 101.5 34.5) (end 98.5 34.5) (stroke (width 0.2) (type default)) (layer "B.Cu") (net 10))
 (gr_line (start 121 56.5) (end 120.5 114) (stroke (width 0.2) (type default)) (layer "B.Cu") (net 18))
 (gr_line (start 113 40) (end 111 38) (stroke (width 0.2) (type default)) (layer "B.Cu") (net 10))
 (gr_line (start 55 42.5) (end 55 49) (stroke (width 0.2) (type default)) (layer "B.Cu") (net 11))
 (gr_line (start 111 38) (end 103.5 38) (stroke (width 0.2) (type default)) (layer "B.Cu") (net 10))
 (gr_line (start 115.5 43) (end 114 43) (stroke (width 0.2) (type default)) (layer "B.Cu") (net 10))
 (gr_line (start 101.5 35.5) (end 101.5 37) (stroke (width 0.2) (type default)) (layer "B.Cu") (net 11))
 (gr_line (start 103.5 38) (end 102.5 37) (stroke (width 0.2) (type default)) (layer "B.Cu") (net 10))
 (gr_line (start 103.5 39) (end 110.5 39) (stroke (width 0.2) (type default)) (layer "B.Cu") (net 11))
 (gr_line (start 110.5 39) (end 111.5 40) (stroke (width 0.2) (type default)) (layer "B.Cu") (net 11))
 (gr_line (start 114 56.5) (end 114 48) (stroke (width 0.2) (type default)) (layer "B.Cu") (net 16))
 (gr_line (start 113 75.5) (end 112 76.5) (stroke (width 0.2) (type default)) (layer "B.Cu") (net 17))
 (gr_line (start 120 55.5) (end 121 56.5) (stroke (width 0.2) (type default)) (layer "B.Cu") (net 18))
 (gr_line (start 98.5 35) (end 101 35) (stroke (width 0.2) (type default)) (layer "B.Cu") (net 11))
 (gr_line (start 96 115) (end 115.5 115) (stroke (width 0.2) (type default)) (layer "B.Cu") (net 18))
 (gr_line (start 111.5 42) (end 112.5 43) (stroke (width 0.2) (type default)) (layer "B.Cu") (net 11))
 (gr_line (start 57.5 50) (end 56 50) (stroke (width 0.2) (type default)) (layer "B.Cu") (net 11))
 (gr_line (start 77 115) (end 58 115) (stroke (width 0.2) (type default)) (layer "B.Cu") (net 18))
 (gr_line (start 100.5 55.5) (end 115.5 55.5) (stroke (width 0.2) (type default)) (layer "B.Cu") (net 17))
 (gr_line (start 101.5 37) (end 103.5 39) (stroke (width 0.2) (type default)) (layer "B.Cu") (net 11))
 (gr_line (start 96 95) (end 77 95) (stroke (width 0.2) (type default)) (layer "B.Cu") (net 16))
 (gr_line (start 54.5 52) (end 54.5 51) (stroke (width 0.2) (type default)) (layer "B.Cu") (net 10))
 (gr_line (start 57 53) (end 56 53) (stroke (width 0.2) (type default)) (layer "B.Cu") (net 10))
 (gr_line (start 56 50) (end 55 49) (stroke (width 0.2) (type default)) (layer "B.Cu") (net 11))
 (gr_line (start 112.5 32) (end 112.5 35.5) (stroke (width 0.05) (type default)) (layer "Edge.Cuts"))
 (gr_line (start 103.5 32) (end 60 32) (stroke (width 0.05) (type default)) (layer "Edge.Cuts"))
 (gr_line (start 122 120) (end 122 122) (stroke (width 0.05) (type default)) (layer "Edge.Cuts"))
 (gr_arc (start 122 122) (mid 120.828427 124.828427) (end 118 126) (stroke (width 0.05) (type default)) (layer "Edge.Cuts"))
 (gr_line (start 117 32) (end 112.5 32) (stroke (width 0.05) (type default)) (layer "Edge.Cuts"))
 (gr_line (start 122.5 37.5) (end 122 120) (stroke (width 0.05) (type default)) (layer "Edge.Cuts"))
 (gr_line (start 103.5 35.5) (end 103.5 32) (stroke (width 0.05) (type default)) (layer "Edge.Cuts"))
 (gr_arc (start 55 126) (mid 52.87868 125.12132) (end 52 123) (stroke (width 0.05) (type default)) (layer "Edge.Cuts"))
 (gr_line (start 55 126) (end 118 126) (stroke (width 0.05) (type default)) (layer "Edge.Cuts"))
 (gr_arc (start 117 32) (mid 120.889087 33.610913) (end 122.5 37.5) (stroke (width 0.05) (type default)) (layer "Edge.Cuts"))
 (gr_line (start 112.5 35.5) (end 103.5 35.5) (stroke (width 0.05) (type default)) (layer "Edge.Cuts"))
 (gr_arc (start 52 40) (mid 54.343146 34.343146) (end 60 32) (stroke (width 0.05) (type default)) (layer "Edge.Cuts"))
 (gr_line (start 52 40) (end 52 123) (stroke (width 0.05) (type default)) (layer "Edge.Cuts"))
 (via (at 118 121) (size 4) (drill 3.4) (layers "F.Cu" "B.Cu") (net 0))
 (via (at 55.5 121.5) (size 4) (drill 3.4) (layers "F.Cu" "B.Cu") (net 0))
 (segment (start 62.73 50.42) (end 57.385 45.075) (width 0.2) (layer "B.Cu") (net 13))
 (segment (start 100.425 50.42) (end 62.73 50.42) (width 0.2) (layer "B.Cu") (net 13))
 (segment (start 54.5 42.434314) (end 62.434314 34.5) (width 0.2) (layer "B.Cu") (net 10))
 (segment (start 54.5 51) (end 54.5 42.434314) (width 0.2) (layer "B.Cu") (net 10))
 (segment (start 98.5 35) (end 62.5 35) (width 0.2) (layer "B.Cu") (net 11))
 (segment (start 62.5 35) (end 55 42.5) (width 0.2) (layer "B.Cu") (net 11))
 (segment (start 57.385 47.615) (end 62.73 52.96) (width 0.2) (layer "B.Cu") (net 12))
 (segment (start 62.73 52.96) (end 100.425 52.96) (width 0.2) (layer "B.Cu") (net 12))
 (segment (start 100.425 42.8) (end 99.34737 42.8) (width 0.2) (layer "F.Cu") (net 8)))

